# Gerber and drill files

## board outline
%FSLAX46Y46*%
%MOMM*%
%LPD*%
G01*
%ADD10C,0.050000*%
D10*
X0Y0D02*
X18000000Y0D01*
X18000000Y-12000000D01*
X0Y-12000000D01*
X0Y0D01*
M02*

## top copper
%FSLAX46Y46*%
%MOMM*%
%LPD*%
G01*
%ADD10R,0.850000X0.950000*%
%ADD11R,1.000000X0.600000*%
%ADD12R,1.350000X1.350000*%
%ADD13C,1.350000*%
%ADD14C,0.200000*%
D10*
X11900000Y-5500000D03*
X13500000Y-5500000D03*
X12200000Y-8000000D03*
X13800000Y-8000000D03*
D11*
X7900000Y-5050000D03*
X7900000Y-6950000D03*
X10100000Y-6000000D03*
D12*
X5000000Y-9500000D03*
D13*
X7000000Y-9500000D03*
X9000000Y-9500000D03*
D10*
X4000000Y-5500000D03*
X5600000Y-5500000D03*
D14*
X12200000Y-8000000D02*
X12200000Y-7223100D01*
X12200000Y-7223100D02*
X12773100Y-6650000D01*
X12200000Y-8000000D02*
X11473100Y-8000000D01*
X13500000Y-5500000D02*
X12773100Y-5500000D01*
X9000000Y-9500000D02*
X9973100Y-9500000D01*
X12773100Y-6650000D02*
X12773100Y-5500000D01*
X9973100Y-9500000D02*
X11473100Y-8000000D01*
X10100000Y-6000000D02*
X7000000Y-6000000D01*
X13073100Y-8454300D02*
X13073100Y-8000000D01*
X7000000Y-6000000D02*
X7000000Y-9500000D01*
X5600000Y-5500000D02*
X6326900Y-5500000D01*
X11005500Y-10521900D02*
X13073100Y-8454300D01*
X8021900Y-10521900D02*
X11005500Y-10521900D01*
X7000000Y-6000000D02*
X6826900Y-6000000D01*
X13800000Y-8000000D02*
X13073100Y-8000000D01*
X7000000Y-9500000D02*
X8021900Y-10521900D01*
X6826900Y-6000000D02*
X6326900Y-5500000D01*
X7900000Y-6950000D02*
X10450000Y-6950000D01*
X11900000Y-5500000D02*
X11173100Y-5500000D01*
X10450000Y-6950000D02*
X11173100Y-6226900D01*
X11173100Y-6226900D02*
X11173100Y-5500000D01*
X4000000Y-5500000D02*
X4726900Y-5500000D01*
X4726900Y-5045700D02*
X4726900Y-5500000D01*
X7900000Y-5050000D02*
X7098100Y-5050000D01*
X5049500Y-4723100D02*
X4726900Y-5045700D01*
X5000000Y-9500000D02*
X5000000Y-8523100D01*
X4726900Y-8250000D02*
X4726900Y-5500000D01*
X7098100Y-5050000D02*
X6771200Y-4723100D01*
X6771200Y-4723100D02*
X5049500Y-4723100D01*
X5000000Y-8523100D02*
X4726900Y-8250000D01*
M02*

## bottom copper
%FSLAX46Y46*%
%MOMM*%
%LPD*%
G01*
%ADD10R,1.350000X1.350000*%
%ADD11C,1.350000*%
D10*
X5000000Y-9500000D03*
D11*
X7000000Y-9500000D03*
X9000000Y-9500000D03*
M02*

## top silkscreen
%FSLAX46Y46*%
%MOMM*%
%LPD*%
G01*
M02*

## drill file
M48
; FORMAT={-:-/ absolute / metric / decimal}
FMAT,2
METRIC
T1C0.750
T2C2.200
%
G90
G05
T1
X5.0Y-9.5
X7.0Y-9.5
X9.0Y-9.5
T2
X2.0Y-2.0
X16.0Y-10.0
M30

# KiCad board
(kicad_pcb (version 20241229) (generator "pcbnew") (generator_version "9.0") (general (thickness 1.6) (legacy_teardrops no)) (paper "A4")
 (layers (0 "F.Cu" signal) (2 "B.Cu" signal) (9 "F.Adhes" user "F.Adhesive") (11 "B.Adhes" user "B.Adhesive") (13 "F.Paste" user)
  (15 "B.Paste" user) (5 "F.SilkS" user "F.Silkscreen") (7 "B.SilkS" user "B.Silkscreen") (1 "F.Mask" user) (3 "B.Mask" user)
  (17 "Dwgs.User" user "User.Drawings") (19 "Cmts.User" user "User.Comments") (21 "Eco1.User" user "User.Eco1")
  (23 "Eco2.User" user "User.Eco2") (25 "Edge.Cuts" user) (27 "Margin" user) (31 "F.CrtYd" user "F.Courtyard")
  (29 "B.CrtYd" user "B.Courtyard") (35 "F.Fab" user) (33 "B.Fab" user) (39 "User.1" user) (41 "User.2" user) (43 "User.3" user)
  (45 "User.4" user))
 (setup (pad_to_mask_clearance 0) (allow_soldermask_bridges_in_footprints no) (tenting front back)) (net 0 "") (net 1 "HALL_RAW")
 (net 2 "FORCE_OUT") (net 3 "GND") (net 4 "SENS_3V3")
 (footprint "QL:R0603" (layer "F.Cu") (at 12.7 5.5)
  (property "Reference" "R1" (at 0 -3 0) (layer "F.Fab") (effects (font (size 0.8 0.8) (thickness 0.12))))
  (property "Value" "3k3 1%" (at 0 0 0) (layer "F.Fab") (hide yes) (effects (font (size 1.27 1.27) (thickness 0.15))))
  (pad "1" smd rect (at -0.8 0) (size 0.85 0.95) (layers "F.Cu" "F.Mask" "F.Paste") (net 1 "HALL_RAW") (thermal_bridge_angle 45))
  (pad "2" smd rect (at 0.8 0) (size 0.85 0.95) (layers "F.Cu" "F.Mask" "F.Paste") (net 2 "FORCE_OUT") (thermal_bridge_angle 45)))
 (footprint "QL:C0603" (layer "F.Cu") (at 13 8)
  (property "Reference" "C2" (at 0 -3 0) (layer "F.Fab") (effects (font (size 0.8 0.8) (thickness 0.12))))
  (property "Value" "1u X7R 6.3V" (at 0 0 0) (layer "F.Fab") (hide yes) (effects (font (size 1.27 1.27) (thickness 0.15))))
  (pad "1" smd rect (at -0.8 0) (size 0.85 0.95) (layers "F.Cu" "F.Mask" "F.Paste") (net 2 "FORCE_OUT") (thermal_bridge_angle 45))
  (pad "2" smd rect (at 0.8 0) (size 0.85 0.95) (layers "F.Cu" "F.Mask" "F.Paste") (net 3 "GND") (thermal_bridge_angle 45)))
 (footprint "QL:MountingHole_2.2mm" (layer "F.Cu") (at 16 10)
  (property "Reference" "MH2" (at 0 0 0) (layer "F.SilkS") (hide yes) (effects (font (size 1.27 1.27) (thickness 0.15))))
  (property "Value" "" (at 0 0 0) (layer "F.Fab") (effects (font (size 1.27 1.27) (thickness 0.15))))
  (pad "" np_thru_hole circle (at 0 0) (size 2.2 2.2) (drill 2.2) (layers "*.Cu" "*.Mask")))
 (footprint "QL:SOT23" (layer "F.Cu") (at 9 6)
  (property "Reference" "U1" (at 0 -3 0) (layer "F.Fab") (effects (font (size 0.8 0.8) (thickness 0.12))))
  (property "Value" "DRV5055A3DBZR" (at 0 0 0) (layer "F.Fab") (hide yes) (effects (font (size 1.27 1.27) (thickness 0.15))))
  (pad "1" smd rect (at -1.1 -0.95) (size 1 0.6) (layers "F.Cu" "F.Mask" "F.Paste") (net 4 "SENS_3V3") (thermal_bridge_angle 45))
  (pad "2" smd rect (at -1.1 0.95) (size 1 0.6) (layers "F.Cu" "F.Mask" "F.Paste") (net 1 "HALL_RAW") (thermal_bridge_angle 45))
  (pad "3" smd rect (at 1.1 0) (size 1 0.6) (layers "F.Cu" "F.Mask" "F.Paste") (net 3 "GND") (thermal_bridge_angle 45)))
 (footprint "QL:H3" (layer "F.Cu") (at 5 9.5)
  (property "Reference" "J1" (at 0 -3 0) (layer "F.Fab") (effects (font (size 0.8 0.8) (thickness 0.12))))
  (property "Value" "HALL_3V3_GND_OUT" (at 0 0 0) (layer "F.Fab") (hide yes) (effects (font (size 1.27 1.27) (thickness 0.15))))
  (pad "1" thru_hole rect (at 0 0) (size 1.35 1.35) (drill 0.75) (layers "*.Cu" "*.Mask") (remove_unused_layers no) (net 4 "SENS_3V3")
   (thermal_bridge_angle 45))
  (pad "2" thru_hole circle (at 2 0) (size 1.35 1.35) (drill 0.75) (layers "*.Cu" "*.Mask") (remove_unused_layers no) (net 3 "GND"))
  (pad "3" thru_hole circle (at 4 0) (size 1.35 1.35) (drill 0.75) (layers "*.Cu" "*.Mask") (remove_unused_layers no) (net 2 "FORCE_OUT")))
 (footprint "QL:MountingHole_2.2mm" (layer "F.Cu") (at 2 2)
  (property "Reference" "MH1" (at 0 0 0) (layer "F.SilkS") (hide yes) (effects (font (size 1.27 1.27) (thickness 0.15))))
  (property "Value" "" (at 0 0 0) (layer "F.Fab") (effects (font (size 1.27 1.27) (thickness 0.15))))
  (pad "" np_thru_hole circle (at 0 0) (size 2.2 2.2) (drill 2.2) (layers "*.Cu" "*.Mask")))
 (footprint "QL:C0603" (layer "F.Cu") (at 4.8 5.5)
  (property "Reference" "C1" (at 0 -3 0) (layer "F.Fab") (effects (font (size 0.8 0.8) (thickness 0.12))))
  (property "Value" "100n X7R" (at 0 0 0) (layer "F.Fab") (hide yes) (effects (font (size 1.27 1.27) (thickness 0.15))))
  (pad "1" smd rect (at -0.8 0) (size 0.85 0.95) (layers "F.Cu" "F.Mask" "F.Paste") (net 4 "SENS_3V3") (thermal_bridge_angle 45))
  (pad "2" smd rect (at 0.8 0) (size 0.85 0.95) (layers "F.Cu" "F.Mask" "F.Paste") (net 3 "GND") (thermal_bridge_angle 45)))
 (gr_rect (start 0 0) (end 18 12) (stroke (width 0.05) (type default)) (fill no) (layer "Edge.Cuts"))
 (segment (start 12.2 8) (end 12.2 7.2231) (width 0.2) (layer "F.Cu") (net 2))
 (segment (start 12.2 7.2231) (end 12.7731 6.65) (width 0.2) (layer "F.Cu") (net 2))
 (segment (start 12.2 8) (end 11.4731 8) (width 0.2) (layer "F.Cu") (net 2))
 (segment (start 13.5 5.5) (end 12.7731 5.5) (width 0.2) (layer "F.Cu") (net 2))
 (segment (start 9 9.5) (end 9.9731 9.5) (width 0.2) (layer "F.Cu") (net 2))
 (segment (start 12.7731 6.65) (end 12.7731 5.5) (width 0.2) (layer "F.Cu") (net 2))
 (segment (start 9.9731 9.5) (end 11.4731 8) (width 0.2) (layer "F.Cu") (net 2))
 (segment (start 10.1 6) (end 7 6) (width 0.2) (layer "F.Cu") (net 3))
 (segment (start 13.0731 8.4543) (end 13.0731 8) (width 0.2) (layer "F.Cu") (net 3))
 (segment (start 7 6) (end 7 9.5) (width 0.2) (layer "F.Cu") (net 3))
 (segment (start 5.6 5.5) (end 6.3269 5.5) (width 0.2) (layer "F.Cu") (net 3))
 (segment (start 11.0055 10.5219) (end 13.0731 8.4543) (width 0.2) (layer "F.Cu") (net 3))
 (segment (start 8.0219 10.5219) (end 11.0055 10.5219) (width 0.2) (layer "F.Cu") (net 3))
 (segment (start 7 6) (end 6.8269 6) (width 0.2) (layer "F.Cu") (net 3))
 (segment (start 13.8 8) (end 13.0731 8) (width 0.2) (layer "F.Cu") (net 3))
 (segment (start 7 9.5) (end 8.0219 10.5219) (width 0.2) (layer "F.Cu") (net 3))
 (segment (start 6.8269 6) (end 6.3269 5.5) (width 0.2) (layer "F.Cu") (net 3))
 (segment (start 7.9 6.95) (end 10.45 6.95) (width 0.2) (layer "F.Cu") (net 1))
 (segment (start 11.9 5.5) (end 11.1731 5.5) (width 0.2) (layer "F.Cu") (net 1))
 (segment (start 10.45 6.95) (end 11.1731 6.2269) (width 0.2) (layer "F.Cu") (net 1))
 (segment (start 11.1731 6.2269) (end 11.1731 5.5) (width 0.2) (layer "F.Cu") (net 1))
 (segment (start 4 5.5) (end 4.7269 5.5) (width 0.2) (layer "F.Cu") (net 4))
 (segment (start 4.7269 5.0457) (end 4.7269 5.5) (width 0.2) (layer "F.Cu") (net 4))
 (segment (start 7.9 5.05) (end 7.0981 5.05) (width 0.2) (layer "F.Cu") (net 4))
 (segment (start 5.0495 4.7231) (end 4.7269 5.0457) (width 0.2) (layer "F.Cu") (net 4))
 (segment (start 5 9.5) (end 5 8.5231) (width 0.2) (layer "F.Cu") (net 4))
 (segment (start 4.7269 8.25) (end 4.7269 5.5) (width 0.2) (layer "F.Cu") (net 4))
 (segment (start 7.0981 5.05) (end 6.7712 4.7231) (width 0.2) (layer "F.Cu") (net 4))
 (segment (start 6.7712 4.7231) (end 5.0495 4.7231) (width 0.2) (layer "F.Cu") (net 4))
 (segment (start 5 8.5231) (end 4.7269 8.25) (width 0.2) (layer "F.Cu") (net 4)))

